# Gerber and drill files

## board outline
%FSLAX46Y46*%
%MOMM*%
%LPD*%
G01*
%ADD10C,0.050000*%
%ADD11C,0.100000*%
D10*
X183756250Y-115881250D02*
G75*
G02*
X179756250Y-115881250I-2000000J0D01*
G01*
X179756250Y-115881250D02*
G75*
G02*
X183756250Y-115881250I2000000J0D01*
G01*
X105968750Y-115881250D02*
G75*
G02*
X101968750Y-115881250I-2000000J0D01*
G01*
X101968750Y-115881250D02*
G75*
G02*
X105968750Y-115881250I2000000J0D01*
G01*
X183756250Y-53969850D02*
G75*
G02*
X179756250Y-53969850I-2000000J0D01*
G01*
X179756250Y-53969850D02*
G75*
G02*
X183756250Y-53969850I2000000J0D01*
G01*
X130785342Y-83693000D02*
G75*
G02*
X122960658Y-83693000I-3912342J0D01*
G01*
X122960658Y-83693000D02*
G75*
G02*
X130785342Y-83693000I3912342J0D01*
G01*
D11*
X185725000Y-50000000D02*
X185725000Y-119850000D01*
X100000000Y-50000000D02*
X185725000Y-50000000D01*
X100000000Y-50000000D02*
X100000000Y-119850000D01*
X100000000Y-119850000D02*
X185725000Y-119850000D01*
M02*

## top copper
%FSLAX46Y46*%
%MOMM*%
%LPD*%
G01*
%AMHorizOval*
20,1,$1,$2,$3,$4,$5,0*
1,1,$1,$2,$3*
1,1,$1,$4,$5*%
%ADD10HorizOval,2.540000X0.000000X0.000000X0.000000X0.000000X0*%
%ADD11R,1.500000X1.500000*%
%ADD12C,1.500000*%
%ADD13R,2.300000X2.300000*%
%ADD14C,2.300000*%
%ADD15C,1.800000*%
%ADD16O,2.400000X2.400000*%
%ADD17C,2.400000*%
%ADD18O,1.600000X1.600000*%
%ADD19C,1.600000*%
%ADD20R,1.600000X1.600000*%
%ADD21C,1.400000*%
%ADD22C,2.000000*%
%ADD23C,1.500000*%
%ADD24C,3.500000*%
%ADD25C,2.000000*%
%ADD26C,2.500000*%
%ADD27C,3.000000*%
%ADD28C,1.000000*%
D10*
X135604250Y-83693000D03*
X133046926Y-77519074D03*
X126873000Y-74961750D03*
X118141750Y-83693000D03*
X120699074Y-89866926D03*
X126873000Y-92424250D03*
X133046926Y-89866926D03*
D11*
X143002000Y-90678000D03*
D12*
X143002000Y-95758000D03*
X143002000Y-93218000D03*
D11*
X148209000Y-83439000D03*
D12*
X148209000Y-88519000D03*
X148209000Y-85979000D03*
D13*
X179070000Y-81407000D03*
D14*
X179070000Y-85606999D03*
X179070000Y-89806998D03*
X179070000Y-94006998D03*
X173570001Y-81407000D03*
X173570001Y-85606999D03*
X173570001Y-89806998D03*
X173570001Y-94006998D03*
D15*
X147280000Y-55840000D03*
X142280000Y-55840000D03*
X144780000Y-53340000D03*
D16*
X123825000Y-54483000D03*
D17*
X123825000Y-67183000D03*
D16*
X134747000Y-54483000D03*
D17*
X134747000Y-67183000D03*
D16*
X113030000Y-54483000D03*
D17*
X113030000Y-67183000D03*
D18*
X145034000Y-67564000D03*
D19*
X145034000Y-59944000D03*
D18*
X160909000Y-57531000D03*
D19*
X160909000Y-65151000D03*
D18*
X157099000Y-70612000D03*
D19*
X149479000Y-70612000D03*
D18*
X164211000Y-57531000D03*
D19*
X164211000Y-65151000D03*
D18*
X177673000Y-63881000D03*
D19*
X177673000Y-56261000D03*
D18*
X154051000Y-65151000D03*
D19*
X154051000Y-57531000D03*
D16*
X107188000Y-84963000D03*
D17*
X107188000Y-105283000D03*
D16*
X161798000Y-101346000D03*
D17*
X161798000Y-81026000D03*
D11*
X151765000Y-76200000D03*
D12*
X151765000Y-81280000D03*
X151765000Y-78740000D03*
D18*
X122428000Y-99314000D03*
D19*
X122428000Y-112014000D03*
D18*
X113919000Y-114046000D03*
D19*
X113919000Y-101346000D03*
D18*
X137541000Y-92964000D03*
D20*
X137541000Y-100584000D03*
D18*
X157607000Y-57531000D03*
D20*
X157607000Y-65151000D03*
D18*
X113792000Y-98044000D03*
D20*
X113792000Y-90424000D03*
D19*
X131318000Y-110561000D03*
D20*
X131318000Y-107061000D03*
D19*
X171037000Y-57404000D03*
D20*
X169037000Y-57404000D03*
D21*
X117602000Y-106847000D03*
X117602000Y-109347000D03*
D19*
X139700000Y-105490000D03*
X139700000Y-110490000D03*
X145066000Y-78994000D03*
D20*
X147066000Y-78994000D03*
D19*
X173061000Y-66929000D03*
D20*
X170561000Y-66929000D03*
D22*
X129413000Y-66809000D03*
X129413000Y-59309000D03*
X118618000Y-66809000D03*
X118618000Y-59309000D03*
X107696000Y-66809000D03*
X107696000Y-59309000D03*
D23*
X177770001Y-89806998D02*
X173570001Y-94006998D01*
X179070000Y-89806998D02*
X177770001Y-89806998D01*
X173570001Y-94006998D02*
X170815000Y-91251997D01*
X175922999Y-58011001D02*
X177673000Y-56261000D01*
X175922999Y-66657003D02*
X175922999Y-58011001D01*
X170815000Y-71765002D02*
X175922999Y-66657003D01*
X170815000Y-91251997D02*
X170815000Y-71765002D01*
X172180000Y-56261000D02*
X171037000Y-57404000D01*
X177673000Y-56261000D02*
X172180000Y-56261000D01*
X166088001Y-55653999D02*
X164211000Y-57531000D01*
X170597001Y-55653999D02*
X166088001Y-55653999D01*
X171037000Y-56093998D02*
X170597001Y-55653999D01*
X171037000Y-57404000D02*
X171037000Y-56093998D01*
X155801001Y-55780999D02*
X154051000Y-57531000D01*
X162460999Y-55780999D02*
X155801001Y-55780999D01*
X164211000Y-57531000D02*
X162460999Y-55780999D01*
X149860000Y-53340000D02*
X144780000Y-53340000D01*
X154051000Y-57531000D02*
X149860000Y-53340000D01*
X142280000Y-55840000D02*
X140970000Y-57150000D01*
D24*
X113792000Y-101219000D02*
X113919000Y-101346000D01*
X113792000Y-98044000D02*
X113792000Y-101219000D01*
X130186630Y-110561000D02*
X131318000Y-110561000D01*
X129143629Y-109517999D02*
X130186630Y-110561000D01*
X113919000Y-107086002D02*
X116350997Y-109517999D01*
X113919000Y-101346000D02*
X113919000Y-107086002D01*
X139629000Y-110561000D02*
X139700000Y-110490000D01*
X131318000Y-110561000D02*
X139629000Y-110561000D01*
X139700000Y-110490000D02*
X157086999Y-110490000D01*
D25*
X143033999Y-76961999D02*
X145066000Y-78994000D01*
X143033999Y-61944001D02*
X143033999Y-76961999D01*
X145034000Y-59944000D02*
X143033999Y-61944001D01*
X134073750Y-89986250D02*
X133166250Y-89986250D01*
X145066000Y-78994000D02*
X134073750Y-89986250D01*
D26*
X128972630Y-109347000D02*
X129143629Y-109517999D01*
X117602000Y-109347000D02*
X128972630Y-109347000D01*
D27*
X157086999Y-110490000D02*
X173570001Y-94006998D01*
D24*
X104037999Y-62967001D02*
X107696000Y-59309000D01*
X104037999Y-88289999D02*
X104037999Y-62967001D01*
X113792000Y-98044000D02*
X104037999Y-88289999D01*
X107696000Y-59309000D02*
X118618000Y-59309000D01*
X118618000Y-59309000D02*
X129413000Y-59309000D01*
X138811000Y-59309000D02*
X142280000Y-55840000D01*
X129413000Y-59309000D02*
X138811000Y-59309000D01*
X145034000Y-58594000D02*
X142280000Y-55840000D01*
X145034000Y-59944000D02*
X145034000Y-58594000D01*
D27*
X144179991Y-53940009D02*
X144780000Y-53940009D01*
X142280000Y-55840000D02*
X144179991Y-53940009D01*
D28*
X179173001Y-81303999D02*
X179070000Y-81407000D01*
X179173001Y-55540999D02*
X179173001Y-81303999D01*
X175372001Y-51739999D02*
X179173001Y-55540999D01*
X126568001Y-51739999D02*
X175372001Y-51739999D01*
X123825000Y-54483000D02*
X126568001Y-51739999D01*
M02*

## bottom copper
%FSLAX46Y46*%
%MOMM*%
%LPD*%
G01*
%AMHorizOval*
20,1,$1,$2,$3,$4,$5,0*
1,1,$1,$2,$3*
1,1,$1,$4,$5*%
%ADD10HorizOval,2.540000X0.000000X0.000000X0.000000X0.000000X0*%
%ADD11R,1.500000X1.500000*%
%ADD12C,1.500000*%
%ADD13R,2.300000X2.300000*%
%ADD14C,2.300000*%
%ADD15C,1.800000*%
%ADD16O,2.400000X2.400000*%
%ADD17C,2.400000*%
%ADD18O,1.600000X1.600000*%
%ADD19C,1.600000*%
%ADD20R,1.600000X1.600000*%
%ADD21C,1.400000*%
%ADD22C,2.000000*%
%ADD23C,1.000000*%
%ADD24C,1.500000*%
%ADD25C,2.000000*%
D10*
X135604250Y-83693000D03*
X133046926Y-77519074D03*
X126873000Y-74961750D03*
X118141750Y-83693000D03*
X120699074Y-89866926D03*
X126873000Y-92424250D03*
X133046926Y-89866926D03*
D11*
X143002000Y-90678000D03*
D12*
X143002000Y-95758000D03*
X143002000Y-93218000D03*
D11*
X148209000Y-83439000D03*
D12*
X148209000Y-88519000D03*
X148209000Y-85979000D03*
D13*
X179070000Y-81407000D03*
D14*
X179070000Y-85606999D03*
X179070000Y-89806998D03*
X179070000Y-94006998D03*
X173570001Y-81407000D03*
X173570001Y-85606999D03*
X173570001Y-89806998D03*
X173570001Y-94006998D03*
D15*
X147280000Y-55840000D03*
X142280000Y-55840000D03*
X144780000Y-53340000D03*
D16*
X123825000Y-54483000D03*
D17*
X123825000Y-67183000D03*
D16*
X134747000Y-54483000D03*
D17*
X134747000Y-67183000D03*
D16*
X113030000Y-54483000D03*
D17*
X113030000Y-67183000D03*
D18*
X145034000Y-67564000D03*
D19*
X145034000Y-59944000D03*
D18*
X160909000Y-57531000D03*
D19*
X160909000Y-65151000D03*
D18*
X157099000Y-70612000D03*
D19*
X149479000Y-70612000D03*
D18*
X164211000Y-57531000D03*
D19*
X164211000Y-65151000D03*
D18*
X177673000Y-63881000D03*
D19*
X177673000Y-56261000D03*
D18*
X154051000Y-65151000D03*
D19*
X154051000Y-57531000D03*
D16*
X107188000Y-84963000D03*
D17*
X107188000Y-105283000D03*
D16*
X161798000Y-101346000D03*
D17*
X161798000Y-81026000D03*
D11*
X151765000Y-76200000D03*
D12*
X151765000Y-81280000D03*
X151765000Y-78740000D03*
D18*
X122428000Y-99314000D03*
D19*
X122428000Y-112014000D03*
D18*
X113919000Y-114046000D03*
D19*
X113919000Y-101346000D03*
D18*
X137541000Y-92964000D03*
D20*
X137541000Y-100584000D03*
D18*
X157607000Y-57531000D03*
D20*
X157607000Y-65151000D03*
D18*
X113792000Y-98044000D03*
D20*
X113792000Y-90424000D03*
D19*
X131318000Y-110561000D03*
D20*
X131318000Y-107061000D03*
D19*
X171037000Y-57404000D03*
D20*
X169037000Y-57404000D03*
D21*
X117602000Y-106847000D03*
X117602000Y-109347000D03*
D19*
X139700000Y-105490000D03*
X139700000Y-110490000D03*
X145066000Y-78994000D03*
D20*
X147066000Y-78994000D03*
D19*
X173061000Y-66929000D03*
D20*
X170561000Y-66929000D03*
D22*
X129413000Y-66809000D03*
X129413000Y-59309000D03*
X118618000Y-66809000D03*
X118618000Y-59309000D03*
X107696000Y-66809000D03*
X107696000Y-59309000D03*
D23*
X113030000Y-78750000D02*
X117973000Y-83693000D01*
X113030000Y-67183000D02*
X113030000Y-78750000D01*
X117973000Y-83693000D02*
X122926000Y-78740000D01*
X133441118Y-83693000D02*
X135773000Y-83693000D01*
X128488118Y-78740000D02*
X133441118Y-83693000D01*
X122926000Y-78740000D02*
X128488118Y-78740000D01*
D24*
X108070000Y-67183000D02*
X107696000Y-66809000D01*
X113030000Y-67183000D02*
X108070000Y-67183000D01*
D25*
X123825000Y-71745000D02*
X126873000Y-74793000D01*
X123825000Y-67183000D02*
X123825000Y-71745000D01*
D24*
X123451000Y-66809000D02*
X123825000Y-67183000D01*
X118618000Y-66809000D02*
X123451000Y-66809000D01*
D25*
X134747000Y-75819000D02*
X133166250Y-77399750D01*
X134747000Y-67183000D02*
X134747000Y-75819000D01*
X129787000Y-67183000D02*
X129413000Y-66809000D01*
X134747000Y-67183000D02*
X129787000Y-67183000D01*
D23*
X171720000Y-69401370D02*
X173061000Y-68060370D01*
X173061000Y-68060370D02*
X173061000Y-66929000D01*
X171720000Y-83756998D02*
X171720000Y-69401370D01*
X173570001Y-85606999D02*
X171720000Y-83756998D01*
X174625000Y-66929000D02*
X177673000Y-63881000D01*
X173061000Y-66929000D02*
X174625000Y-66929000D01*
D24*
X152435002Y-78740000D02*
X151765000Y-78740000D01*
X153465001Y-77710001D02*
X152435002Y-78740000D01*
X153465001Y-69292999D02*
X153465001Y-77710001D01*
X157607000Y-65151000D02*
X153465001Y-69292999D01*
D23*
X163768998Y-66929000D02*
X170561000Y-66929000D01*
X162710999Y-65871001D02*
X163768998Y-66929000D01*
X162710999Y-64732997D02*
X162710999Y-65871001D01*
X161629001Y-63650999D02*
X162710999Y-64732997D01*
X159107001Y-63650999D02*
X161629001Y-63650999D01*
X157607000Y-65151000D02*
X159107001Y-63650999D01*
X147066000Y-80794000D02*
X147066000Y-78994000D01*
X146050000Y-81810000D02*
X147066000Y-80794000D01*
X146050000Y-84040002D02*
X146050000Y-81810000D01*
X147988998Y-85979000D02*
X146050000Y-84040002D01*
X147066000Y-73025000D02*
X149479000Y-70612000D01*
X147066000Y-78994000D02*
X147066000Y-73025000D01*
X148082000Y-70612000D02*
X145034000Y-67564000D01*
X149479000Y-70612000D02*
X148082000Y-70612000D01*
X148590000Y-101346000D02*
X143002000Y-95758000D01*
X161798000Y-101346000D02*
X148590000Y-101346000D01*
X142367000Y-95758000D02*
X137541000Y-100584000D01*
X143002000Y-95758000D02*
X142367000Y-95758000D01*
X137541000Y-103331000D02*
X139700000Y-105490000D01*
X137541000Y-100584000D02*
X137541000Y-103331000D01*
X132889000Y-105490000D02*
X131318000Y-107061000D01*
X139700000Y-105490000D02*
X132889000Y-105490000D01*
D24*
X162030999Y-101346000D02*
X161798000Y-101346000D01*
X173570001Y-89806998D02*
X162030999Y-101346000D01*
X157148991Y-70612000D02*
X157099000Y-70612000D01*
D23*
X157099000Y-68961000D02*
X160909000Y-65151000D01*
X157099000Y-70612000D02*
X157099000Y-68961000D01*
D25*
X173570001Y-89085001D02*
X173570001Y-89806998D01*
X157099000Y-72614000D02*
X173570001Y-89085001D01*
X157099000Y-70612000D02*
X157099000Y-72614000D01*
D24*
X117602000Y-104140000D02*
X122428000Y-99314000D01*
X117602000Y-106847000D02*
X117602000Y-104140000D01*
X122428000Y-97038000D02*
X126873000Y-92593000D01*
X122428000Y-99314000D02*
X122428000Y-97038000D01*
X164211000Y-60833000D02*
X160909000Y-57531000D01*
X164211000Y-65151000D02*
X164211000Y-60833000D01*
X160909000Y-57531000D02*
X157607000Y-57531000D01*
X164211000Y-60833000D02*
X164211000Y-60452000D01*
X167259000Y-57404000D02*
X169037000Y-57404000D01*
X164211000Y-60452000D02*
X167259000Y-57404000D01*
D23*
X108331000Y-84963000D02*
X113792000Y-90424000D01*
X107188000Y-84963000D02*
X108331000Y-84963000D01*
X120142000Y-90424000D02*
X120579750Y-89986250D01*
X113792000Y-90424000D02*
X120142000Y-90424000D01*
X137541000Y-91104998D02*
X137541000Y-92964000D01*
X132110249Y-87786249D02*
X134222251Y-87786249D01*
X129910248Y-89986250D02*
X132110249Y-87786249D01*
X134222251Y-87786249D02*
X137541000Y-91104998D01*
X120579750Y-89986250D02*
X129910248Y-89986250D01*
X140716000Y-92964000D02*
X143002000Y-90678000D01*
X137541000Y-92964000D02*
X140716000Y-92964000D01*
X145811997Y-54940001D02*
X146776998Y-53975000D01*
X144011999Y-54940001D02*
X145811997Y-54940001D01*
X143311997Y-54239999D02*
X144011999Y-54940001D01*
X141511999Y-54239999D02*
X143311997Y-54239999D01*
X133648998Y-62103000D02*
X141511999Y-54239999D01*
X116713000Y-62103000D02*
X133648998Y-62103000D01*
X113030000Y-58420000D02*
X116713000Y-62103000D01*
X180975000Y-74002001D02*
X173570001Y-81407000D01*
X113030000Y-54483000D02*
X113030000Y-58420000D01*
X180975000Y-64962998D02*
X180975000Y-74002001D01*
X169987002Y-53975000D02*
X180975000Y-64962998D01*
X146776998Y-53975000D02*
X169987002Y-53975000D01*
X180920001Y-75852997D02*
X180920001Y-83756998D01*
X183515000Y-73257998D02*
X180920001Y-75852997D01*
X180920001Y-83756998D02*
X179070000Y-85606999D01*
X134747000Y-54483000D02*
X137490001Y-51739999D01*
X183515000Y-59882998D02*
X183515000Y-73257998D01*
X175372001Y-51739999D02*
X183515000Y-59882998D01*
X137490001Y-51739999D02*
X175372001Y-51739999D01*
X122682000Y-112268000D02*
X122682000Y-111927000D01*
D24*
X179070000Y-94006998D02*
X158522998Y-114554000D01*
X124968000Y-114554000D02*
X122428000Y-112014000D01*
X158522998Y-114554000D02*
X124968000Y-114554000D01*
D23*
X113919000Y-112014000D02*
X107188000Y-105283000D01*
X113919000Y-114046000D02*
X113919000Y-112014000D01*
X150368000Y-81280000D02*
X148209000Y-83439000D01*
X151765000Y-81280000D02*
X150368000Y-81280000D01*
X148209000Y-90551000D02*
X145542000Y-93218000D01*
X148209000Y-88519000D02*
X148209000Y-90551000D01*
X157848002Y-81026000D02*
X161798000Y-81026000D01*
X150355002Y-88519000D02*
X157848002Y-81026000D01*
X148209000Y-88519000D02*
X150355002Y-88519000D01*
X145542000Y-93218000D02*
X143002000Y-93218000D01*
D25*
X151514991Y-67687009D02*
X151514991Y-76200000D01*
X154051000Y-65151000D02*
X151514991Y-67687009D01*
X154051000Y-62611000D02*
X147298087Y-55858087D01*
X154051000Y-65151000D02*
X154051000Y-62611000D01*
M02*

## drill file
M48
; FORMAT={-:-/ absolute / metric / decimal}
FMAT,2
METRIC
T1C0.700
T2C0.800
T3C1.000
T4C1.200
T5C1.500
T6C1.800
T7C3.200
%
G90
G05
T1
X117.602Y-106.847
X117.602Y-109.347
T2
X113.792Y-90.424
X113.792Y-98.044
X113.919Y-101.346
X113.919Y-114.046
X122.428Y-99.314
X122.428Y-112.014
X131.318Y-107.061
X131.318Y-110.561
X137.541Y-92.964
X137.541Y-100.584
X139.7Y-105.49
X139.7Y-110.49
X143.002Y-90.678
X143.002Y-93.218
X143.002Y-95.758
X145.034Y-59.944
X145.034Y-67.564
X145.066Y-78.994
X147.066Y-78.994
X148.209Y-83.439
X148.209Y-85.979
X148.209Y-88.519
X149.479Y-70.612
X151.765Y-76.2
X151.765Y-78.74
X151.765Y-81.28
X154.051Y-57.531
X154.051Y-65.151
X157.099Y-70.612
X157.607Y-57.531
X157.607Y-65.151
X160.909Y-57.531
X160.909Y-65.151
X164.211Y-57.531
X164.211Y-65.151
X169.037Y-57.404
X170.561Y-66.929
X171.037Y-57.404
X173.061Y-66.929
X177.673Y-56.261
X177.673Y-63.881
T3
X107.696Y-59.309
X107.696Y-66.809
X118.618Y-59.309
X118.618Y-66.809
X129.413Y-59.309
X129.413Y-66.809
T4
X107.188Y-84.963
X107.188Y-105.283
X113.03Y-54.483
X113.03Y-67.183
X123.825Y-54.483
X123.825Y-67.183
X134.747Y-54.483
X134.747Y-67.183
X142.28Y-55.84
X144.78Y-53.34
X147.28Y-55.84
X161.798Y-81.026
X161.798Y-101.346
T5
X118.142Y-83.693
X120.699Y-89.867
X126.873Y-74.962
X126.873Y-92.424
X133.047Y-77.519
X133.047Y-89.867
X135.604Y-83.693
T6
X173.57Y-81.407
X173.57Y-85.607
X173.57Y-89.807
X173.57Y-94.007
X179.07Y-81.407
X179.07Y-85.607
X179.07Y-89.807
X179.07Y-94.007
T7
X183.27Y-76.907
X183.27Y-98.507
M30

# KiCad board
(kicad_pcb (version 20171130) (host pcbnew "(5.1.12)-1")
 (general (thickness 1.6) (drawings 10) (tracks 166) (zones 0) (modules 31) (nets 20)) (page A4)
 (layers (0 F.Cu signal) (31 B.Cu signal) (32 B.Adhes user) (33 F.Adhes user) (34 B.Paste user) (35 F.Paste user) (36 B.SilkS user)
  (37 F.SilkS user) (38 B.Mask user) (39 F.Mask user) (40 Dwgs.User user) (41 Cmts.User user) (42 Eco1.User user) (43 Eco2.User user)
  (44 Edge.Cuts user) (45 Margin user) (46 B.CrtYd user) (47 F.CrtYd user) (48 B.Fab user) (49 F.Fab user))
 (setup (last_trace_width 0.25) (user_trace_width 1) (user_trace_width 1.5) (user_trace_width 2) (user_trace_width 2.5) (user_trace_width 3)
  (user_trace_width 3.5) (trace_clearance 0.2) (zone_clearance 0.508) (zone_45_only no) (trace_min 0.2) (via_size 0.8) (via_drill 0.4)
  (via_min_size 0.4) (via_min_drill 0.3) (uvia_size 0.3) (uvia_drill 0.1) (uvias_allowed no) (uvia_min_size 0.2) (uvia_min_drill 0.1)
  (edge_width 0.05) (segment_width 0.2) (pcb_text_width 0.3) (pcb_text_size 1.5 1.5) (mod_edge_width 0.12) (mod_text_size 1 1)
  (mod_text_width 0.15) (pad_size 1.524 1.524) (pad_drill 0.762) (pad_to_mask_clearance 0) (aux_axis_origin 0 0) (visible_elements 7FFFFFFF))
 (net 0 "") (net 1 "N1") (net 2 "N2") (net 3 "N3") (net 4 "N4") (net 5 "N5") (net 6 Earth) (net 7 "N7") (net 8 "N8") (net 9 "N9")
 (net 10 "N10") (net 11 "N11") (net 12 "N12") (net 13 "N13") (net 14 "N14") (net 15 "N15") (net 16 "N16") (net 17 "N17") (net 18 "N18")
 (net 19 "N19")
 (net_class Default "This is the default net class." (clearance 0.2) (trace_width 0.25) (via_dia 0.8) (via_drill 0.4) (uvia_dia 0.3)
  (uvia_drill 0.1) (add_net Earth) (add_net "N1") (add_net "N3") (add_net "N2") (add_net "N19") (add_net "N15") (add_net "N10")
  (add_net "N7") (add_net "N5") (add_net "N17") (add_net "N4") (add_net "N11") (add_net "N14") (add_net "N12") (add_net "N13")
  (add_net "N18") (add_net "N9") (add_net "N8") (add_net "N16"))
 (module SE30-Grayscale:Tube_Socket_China (layer F.Cu) (at 126.873 83.693 225)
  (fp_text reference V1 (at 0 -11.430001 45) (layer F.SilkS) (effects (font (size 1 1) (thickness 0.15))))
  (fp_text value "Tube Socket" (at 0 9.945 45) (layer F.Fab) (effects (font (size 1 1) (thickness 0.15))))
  (pad 5 thru_hole oval (at -6.173926 -6.173926 225) (size 2.54 2.54) (drill 1.5) (layers *.Cu *.Mask) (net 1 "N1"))
  (pad 6 thru_hole oval (at -8.73125 0 225) (size 2.54 2.54) (drill 1.5) (layers *.Cu *.Mask) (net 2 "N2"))
  (pad 7 thru_hole oval (at -6.173926 6.173926 225) (size 2.54 2.54) (drill 1.5) (layers *.Cu *.Mask) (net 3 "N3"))
  (pad 1 thru_hole oval (at 6.173926 6.173926 225) (size 2.54 2.54) (drill 1.5) (layers *.Cu *.Mask) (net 1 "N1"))
  (pad 2 thru_hole oval (at 8.73125 0 225) (size 2.54 2.54) (drill 1.5) (layers *.Cu *.Mask) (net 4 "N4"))
  (pad 3 thru_hole oval (at 6.173926 -6.173926 225) (size 2.54 2.54) (drill 1.5) (layers *.Cu *.Mask) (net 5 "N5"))
  (pad 4 thru_hole oval (at 0 -8.73125 225) (size 2.54 2.54) (drill 1.5) (layers *.Cu *.Mask) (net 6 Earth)))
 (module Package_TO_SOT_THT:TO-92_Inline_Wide (layer F.Cu) (at 143.002 90.678 270)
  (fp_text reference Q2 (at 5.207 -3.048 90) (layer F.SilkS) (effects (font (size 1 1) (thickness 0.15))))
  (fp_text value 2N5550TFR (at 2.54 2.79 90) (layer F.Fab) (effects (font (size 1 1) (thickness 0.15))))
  (pad 1 thru_hole rect (at 0 0 270) (size 1.5 1.5) (drill 0.8) (layers *.Cu *.Mask) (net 4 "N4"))
  (pad 3 thru_hole circle (at 5.08 0 270) (size 1.5 1.5) (drill 0.8) (layers *.Cu *.Mask) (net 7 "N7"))
  (pad 2 thru_hole circle (at 2.54 0 270) (size 1.5 1.5) (drill 0.8) (layers *.Cu *.Mask) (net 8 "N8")))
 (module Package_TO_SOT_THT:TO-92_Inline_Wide (layer F.Cu) (at 148.209 83.439 270)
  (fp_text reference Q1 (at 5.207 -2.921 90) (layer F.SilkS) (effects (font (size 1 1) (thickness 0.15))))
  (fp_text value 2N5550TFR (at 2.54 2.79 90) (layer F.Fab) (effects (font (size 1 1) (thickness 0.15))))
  (pad 1 thru_hole rect (at 0 0 270) (size 1.5 1.5) (drill 0.8) (layers *.Cu *.Mask) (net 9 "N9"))
  (pad 3 thru_hole circle (at 5.08 0 270) (size 1.5 1.5) (drill 0.8) (layers *.Cu *.Mask) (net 8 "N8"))
  (pad 2 thru_hole circle (at 2.54 0 270) (size 1.5 1.5) (drill 0.8) (layers *.Cu *.Mask) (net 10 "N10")))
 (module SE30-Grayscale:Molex (layer F.Cu) (at 179.07 81.407 90)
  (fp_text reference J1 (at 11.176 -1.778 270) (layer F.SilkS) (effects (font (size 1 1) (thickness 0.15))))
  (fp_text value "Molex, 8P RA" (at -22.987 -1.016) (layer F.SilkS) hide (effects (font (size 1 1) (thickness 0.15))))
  (pad 1 thru_hole rect (at 0 0 90) (size 2.3 2.3) (drill 1.8) (layers *.Cu *.Mask) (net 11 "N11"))
  (pad 3 thru_hole circle (at -4.199999 0 90) (size 2.3 2.3) (drill 1.8) (layers *.Cu *.Mask) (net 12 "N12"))
  (pad 5 thru_hole circle (at -8.399998 0 90) (size 2.3 2.3) (drill 1.8) (layers *.Cu *.Mask) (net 6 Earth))
  (pad 7 thru_hole circle (at -12.599998 0 90) (size 2.3 2.3) (drill 1.8) (layers *.Cu *.Mask) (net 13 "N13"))
  (pad 2 thru_hole circle (at 0 -5.499999 90) (size 2.3 2.3) (drill 1.8) (layers *.Cu *.Mask) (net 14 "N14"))
  (pad 4 thru_hole circle (at -4.199999 -5.499999 90) (size 2.3 2.3) (drill 1.8) (layers *.Cu *.Mask) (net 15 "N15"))
  (pad 6 thru_hole circle (at -8.399998 -5.499999 90) (size 2.3 2.3) (drill 1.8) (layers *.Cu *.Mask) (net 7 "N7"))
  (pad 8 thru_hole circle (at -12.599998 -5.499999 90) (size 2.3 2.3) (drill 1.8) (layers *.Cu *.Mask) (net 6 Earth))
  (pad M1 np_thru_hole circle (at 4.499999 4.199999 90) (size 3.200001 3.200001) (drill 3.200001) (layers *.Cu *.Mask))
  (pad M2 np_thru_hole circle (at -17.099958 4.199999 90) (size 3.200001 3.200001) (drill 3.200001) (layers *.Cu *.Mask)))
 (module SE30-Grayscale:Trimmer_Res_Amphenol (layer F.Cu) (at 144.78 53.34)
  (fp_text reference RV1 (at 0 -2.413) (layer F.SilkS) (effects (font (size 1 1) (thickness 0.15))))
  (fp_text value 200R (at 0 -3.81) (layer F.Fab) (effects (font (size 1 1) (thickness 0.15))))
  (pad 3 thru_hole circle (at 2.5 2.5) (size 1.8 1.8) (drill 1.2) (layers *.Cu *.Mask) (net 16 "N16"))
  (pad 1 thru_hole circle (at -2.5 2.5) (size 1.8 1.8) (drill 1.2) (layers *.Cu *.Mask) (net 6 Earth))
  (pad 2 thru_hole circle (at 0 0) (size 1.8 1.8) (drill 1.2) (layers *.Cu *.Mask) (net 6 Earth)))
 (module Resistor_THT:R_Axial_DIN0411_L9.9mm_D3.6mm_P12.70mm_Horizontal (layer F.Cu) (at 123.825 67.183 90)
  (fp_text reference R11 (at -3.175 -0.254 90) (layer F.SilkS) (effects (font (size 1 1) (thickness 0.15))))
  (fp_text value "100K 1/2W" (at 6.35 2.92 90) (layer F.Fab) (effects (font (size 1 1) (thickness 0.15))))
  (pad 2 thru_hole oval (at 12.7 0 90) (size 2.4 2.4) (drill 1.2) (layers *.Cu *.Mask) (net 11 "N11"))
  (pad 1 thru_hole circle (at 0 0 90) (size 2.4 2.4) (drill 1.2) (layers *.Cu *.Mask) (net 3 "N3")))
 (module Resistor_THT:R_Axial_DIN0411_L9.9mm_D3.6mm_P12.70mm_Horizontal (layer F.Cu) (at 134.747 67.183 90)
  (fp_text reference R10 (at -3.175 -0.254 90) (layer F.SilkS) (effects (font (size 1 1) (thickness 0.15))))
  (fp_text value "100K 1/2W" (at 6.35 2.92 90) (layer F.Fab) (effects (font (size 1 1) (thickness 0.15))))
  (pad 2 thru_hole oval (at 12.7 0 90) (size 2.4 2.4) (drill 1.2) (layers *.Cu *.Mask) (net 12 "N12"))
  (pad 1 thru_hole circle (at 0 0 90) (size 2.4 2.4) (drill 1.2) (layers *.Cu *.Mask) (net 2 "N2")))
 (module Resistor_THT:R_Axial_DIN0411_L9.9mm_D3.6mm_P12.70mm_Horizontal (layer F.Cu) (at 113.03 67.183 90)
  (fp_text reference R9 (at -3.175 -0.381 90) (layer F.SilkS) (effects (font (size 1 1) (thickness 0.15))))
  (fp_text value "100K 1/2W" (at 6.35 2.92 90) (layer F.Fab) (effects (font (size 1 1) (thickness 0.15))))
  (pad 2 thru_hole oval (at 12.7 0 90) (size 2.4 2.4) (drill 1.2) (layers *.Cu *.Mask) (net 14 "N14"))
  (pad 1 thru_hole circle (at 0 0 90) (size 2.4 2.4) (drill 1.2) (layers *.Cu *.Mask) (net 1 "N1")))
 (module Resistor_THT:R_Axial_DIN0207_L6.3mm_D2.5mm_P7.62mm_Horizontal (layer F.Cu) (at 145.034 59.944 270)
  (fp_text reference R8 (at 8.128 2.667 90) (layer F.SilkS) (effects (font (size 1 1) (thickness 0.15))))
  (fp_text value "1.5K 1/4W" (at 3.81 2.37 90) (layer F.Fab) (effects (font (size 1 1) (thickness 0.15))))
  (pad 2 thru_hole oval (at 7.62 0 270) (size 1.6 1.6) (drill 0.8) (layers *.Cu *.Mask) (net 10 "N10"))
  (pad 1 thru_hole circle (at 0 0 270) (size 1.6 1.6) (drill 0.8) (layers *.Cu *.Mask) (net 6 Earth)))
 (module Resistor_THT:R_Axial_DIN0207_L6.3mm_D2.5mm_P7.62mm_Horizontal (layer F.Cu) (at 160.909 65.151 90)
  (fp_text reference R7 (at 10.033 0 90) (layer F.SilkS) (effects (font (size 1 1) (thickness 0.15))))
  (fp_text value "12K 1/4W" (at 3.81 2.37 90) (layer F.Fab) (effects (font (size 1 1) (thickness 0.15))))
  (pad 2 thru_hole oval (at 7.62 0 90) (size 1.6 1.6) (drill 0.8) (layers *.Cu *.Mask) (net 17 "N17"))
  (pad 1 thru_hole circle (at 0 0 90) (size 1.6 1.6) (drill 0.8) (layers *.Cu *.Mask) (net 7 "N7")))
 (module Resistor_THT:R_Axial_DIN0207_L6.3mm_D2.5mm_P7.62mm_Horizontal (layer F.Cu) (at 149.479 70.612)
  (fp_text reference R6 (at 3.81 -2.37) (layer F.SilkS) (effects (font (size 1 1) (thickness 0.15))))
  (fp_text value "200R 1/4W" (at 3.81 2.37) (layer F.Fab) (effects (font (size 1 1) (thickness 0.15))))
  (pad 2 thru_hole oval (at 7.62 0) (size 1.6 1.6) (drill 0.8) (layers *.Cu *.Mask) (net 7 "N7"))
  (pad 1 thru_hole circle (at 0 0) (size 1.6 1.6) (drill 0.8) (layers *.Cu *.Mask) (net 10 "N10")))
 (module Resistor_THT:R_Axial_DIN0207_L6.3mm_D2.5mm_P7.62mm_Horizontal (layer F.Cu) (at 164.211 65.151 90)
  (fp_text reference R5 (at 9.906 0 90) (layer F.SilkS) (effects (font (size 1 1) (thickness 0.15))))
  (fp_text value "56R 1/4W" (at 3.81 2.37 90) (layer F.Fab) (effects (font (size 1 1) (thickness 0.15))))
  (pad 2 thru_hole oval (at 7.62 0 90) (size 1.6 1.6) (drill 0.8) (layers *.Cu *.Mask) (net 6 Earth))
  (pad 1 thru_hole circle (at 0 0 90) (size 1.6 1.6) (drill 0.8) (layers *.Cu *.Mask) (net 17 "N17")))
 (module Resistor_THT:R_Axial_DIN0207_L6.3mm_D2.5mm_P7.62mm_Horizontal (layer F.Cu) (at 177.673 56.261 270)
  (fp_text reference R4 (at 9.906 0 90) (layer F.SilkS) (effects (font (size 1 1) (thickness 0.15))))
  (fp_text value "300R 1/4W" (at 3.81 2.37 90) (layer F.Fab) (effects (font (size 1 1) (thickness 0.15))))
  (pad 2 thru_hole oval (at 7.62 0 270) (size 1.6 1.6) (drill 0.8) (layers *.Cu *.Mask) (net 15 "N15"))
  (pad 1 thru_hole circle (at 0 0 270) (size 1.6 1.6) (drill 0.8) (layers *.Cu *.Mask) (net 6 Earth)))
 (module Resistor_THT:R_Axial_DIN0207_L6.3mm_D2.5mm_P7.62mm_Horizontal (layer F.Cu) (at 154.051 57.531 270)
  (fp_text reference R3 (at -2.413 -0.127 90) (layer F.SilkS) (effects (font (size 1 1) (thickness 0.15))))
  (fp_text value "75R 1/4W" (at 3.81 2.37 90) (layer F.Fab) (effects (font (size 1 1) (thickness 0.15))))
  (pad 2 thru_hole oval (at 7.62 0 270) (size 1.6 1.6) (drill 0.8) (layers *.Cu *.Mask) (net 16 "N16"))
  (pad 1 thru_hole circle (at 0 0 270) (size 1.6 1.6) (drill 0.8) (layers *.Cu *.Mask) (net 6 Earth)))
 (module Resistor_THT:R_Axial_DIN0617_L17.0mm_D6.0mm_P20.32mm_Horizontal (layer F.Cu) (at 107.188 105.283 90)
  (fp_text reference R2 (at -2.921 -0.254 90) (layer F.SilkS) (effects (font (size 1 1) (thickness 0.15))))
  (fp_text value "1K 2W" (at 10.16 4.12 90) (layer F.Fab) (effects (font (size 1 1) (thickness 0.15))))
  (pad 2 thru_hole oval (at 20.32 0 90) (size 2.4 2.4) (drill 1.2) (layers *.Cu *.Mask) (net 4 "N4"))
  (pad 1 thru_hole circle (at 0 0 90) (size 2.4 2.4) (drill 1.2) (layers *.Cu *.Mask) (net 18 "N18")))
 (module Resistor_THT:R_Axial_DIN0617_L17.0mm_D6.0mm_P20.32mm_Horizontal (layer F.Cu) (at 161.798 81.026 270)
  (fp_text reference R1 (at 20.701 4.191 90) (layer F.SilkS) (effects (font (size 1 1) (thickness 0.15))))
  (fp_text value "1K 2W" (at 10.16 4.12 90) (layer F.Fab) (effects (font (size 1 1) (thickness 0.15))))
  (pad 2 thru_hole oval (at 20.32 0 270) (size 2.4 2.4) (drill 1.2) (layers *.Cu *.Mask) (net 7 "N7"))
  (pad 1 thru_hole circle (at 0 0 270) (size 2.4 2.4) (drill 1.2) (layers *.Cu *.Mask) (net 8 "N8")))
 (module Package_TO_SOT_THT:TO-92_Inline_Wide (layer F.Cu) (at 151.765 76.2 270)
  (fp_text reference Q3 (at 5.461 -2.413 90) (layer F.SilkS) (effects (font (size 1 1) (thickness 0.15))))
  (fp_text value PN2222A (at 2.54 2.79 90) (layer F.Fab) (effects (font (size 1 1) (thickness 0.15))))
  (pad 1 thru_hole rect (at 0 0 270) (size 1.5 1.5) (drill 0.8) (layers *.Cu *.Mask) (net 16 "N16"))
  (pad 3 thru_hole circle (at 5.08 0 270) (size 1.5 1.5) (drill 0.8) (layers *.Cu *.Mask) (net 9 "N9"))
  (pad 2 thru_hole circle (at 2.54 0 270) (size 1.5 1.5) (drill 0.8) (layers *.Cu *.Mask) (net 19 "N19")))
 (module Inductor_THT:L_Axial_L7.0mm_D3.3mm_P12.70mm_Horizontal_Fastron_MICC (layer F.Cu) (at 122.428 112.014 90)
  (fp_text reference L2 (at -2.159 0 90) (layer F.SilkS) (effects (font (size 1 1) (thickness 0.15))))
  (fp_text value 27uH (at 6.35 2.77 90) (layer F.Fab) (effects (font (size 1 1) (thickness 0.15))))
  (pad 2 thru_hole oval (at 12.7 0 90) (size 1.6 1.6) (drill 0.8) (layers *.Cu *.Mask) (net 5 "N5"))
  (pad 1 thru_hole circle (at 0 0 90) (size 1.6 1.6) (drill 0.8) (layers *.Cu *.Mask) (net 13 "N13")))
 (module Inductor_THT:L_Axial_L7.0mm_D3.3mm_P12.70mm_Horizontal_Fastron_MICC (layer F.Cu) (at 113.919 101.346 270)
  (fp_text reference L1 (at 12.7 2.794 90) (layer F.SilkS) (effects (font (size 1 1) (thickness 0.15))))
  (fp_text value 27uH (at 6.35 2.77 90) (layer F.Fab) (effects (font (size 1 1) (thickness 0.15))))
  (pad 2 thru_hole oval (at 12.7 0 270) (size 1.6 1.6) (drill 0.8) (layers *.Cu *.Mask) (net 18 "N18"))
  (pad 1 thru_hole circle (at 0 0 270) (size 1.6 1.6) (drill 0.8) (layers *.Cu *.Mask) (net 6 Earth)))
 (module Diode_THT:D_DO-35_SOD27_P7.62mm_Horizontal (layer F.Cu) (at 137.541 100.584 90)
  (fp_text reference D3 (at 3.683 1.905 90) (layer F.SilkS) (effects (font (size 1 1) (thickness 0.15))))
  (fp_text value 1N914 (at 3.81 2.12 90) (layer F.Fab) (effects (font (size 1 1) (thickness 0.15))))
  (pad 2 thru_hole oval (at 7.62 0 90) (size 1.6 1.6) (drill 0.8) (layers *.Cu *.Mask) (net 4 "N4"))
  (pad 1 thru_hole rect (at 0 0 90) (size 1.6 1.6) (drill 0.8) (layers *.Cu *.Mask) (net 7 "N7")))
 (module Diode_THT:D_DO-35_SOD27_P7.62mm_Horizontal (layer F.Cu) (at 157.607 65.151 90)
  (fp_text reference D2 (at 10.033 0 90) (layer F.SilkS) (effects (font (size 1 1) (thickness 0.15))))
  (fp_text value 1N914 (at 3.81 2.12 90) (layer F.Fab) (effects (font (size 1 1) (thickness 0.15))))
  (pad 2 thru_hole oval (at 7.62 0 90) (size 1.6 1.6) (drill 0.8) (layers *.Cu *.Mask) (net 17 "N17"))
  (pad 1 thru_hole rect (at 0 0 90) (size 1.6 1.6) (drill 0.8) (layers *.Cu *.Mask) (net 19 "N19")))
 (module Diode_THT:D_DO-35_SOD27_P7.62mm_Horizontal (layer F.Cu) (at 113.792 90.424 270)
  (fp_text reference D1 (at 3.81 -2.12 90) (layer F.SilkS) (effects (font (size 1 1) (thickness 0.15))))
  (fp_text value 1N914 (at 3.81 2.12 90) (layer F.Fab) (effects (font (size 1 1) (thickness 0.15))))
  (pad 2 thru_hole oval (at 7.62 0 270) (size 1.6 1.6) (drill 0.8) (layers *.Cu *.Mask) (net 6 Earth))
  (pad 1 thru_hole rect (at 0 0 270) (size 1.6 1.6) (drill 0.8) (layers *.Cu *.Mask) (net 4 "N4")))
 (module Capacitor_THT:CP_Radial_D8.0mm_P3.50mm (layer F.Cu) (at 131.318 107.061 270)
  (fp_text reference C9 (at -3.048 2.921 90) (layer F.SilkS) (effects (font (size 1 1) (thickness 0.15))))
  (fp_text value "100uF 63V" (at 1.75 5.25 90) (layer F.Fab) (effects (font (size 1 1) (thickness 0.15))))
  (pad 2 thru_hole circle (at 3.5 0 270) (size 1.6 1.6) (drill 0.8) (layers *.Cu *.Mask) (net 6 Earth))
  (pad 1 thru_hole rect (at 0 0 270) (size 1.6 1.6) (drill 0.8) (layers *.Cu *.Mask) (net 7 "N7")))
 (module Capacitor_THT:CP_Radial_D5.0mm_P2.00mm (layer F.Cu) (at 169.037 57.404)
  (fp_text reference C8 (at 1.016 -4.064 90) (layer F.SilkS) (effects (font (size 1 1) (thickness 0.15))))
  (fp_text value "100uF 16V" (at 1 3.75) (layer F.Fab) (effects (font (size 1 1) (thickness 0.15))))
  (pad 2 thru_hole circle (at 2 0) (size 1.6 1.6) (drill 0.8) (layers *.Cu *.Mask) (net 6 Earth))
  (pad 1 thru_hole rect (at 0 0) (size 1.6 1.6) (drill 0.8) (layers *.Cu *.Mask) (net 17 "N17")))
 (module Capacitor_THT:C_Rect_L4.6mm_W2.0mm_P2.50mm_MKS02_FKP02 (layer F.Cu) (at 117.602 109.347 90)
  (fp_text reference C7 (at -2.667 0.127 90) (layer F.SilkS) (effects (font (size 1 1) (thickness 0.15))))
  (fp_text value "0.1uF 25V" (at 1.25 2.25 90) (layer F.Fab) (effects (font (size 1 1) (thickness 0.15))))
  (pad 2 thru_hole circle (at 2.5 0 90) (size 1.4 1.4) (drill 0.7) (layers *.Cu *.Mask) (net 5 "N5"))
  (pad 1 thru_hole circle (at 0 0 90) (size 1.4 1.4) (drill 0.7) (layers *.Cu *.Mask) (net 6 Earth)))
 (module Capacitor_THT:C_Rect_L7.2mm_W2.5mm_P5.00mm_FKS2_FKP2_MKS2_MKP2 (layer F.Cu) (at 139.7 110.49 90)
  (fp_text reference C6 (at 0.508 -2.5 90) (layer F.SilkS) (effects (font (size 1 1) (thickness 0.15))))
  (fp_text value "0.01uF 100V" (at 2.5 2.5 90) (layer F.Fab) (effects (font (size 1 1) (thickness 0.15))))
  (pad 2 thru_hole circle (at 5 0 90) (size 1.6 1.6) (drill 0.8) (layers *.Cu *.Mask) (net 7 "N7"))
  (pad 1 thru_hole circle (at 0 0 90) (size 1.6 1.6) (drill 0.8) (layers *.Cu *.Mask) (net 6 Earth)))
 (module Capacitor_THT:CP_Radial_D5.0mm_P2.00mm (layer F.Cu) (at 147.066 78.994 180)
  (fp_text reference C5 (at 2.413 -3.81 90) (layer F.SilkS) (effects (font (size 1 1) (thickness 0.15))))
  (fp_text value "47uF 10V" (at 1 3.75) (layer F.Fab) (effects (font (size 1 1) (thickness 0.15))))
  (pad 2 thru_hole circle (at 2 0 180) (size 1.6 1.6) (drill 0.8) (layers *.Cu *.Mask) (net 6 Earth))
  (pad 1 thru_hole rect (at 0 0 180) (size 1.6 1.6) (drill 0.8) (layers *.Cu *.Mask) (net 10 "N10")))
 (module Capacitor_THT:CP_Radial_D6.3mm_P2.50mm (layer F.Cu) (at 170.561 66.929)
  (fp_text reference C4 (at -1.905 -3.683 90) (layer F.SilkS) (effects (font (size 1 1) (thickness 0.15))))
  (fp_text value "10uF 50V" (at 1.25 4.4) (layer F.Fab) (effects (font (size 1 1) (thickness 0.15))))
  (pad 2 thru_hole circle (at 2.5 0) (size 1.6 1.6) (drill 0.8) (layers *.Cu *.Mask) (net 15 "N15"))
  (pad 1 thru_hole rect (at 0 0) (size 1.6 1.6) (drill 0.8) (layers *.Cu *.Mask) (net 19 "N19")))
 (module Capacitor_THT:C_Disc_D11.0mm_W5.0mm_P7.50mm (layer F.Cu) (at 129.413 59.309 270)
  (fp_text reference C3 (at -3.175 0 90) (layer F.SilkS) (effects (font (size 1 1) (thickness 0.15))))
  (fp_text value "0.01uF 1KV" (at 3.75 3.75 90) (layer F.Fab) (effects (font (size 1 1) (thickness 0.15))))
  (pad 2 thru_hole circle (at 7.5 0 270) (size 2 2) (drill 1) (layers *.Cu *.Mask) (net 2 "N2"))
  (pad 1 thru_hole circle (at 0 0 270) (size 2 2) (drill 1) (layers *.Cu *.Mask) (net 6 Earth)))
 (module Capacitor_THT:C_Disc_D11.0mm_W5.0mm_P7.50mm (layer F.Cu) (at 118.618 59.309 270)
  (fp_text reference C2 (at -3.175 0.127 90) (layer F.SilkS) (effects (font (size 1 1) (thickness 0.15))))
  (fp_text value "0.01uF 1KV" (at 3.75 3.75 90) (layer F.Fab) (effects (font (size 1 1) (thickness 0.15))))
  (pad 2 thru_hole circle (at 7.5 0 270) (size 2 2) (drill 1) (layers *.Cu *.Mask) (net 3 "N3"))
  (pad 1 thru_hole circle (at 0 0 270) (size 2 2) (drill 1) (layers *.Cu *.Mask) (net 6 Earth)))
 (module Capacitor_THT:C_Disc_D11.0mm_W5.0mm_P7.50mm (layer F.Cu) (at 107.696 59.309 270)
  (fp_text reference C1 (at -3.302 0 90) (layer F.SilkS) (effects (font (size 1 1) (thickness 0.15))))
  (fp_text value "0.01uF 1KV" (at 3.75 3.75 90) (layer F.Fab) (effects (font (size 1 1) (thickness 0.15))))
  (pad 2 thru_hole circle (at 7.5 0 270) (size 2 2) (drill 1) (layers *.Cu *.Mask) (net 1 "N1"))
  (pad 1 thru_hole circle (at 0 0 270) (size 2 2) (drill 1) (layers *.Cu *.Mask) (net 6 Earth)))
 (gr_circle (center 181.75625 115.88125) (end 183.75625 115.88125) (layer Edge.Cuts) (width 0.05))
 (gr_circle (center 103.96875 115.88125) (end 105.96875 115.88125) (layer Edge.Cuts) (width 0.05))
 (gr_circle (center 181.75625 53.96985) (end 183.75625 53.96985) (layer Edge.Cuts) (width 0.05))
 (gr_circle (center 126.873 83.693) (end 130.785342 83.693) (layer Edge.Cuts) (width 0.05))
 (gr_line (start 185.725 50) (end 185.725 119.85) (layer Edge.Cuts) (width 0.1))
 (gr_line (start 100 50) (end 185.725 50) (layer Edge.Cuts) (width 0.1))
 (gr_line (start 100 50) (end 100 119.85) (layer Edge.Cuts) (width 0.1))
 (gr_line (start 100 119.85) (end 185.725 119.85) (layer Edge.Cuts) (width 0.1))
 (segment (start 113.03 78.75) (end 117.973 83.693) (width 1) (layer B.Cu) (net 1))
 (segment (start 113.03 67.183) (end 113.03 78.75) (width 1) (layer B.Cu) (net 1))
 (segment (start 117.973 83.693) (end 122.926 78.74) (width 1) (layer B.Cu) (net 1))
 (segment (start 133.441118 83.693) (end 135.773 83.693) (width 1) (layer B.Cu) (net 1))
 (segment (start 128.488118 78.74) (end 133.441118 83.693) (width 1) (layer B.Cu) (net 1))
 (segment (start 122.926 78.74) (end 128.488118 78.74) (width 1) (layer B.Cu) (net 1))
 (segment (start 108.07 67.183) (end 107.696 66.809) (width 1.5) (layer B.Cu) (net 1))
 (segment (start 113.03 67.183) (end 108.07 67.183) (width 1.5) (layer B.Cu) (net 1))
 (segment (start 177.770001 89.806998) (end 173.570001 94.006998) (width 1.5) (layer F.Cu) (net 6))
 (segment (start 179.07 89.806998) (end 177.770001 89.806998) (width 1.5) (layer F.Cu) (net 6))
 (segment (start 173.570001 94.006998) (end 170.815 91.251997) (width 1.5) (layer F.Cu) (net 6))
 (segment (start 175.922999 58.011001) (end 177.673 56.261) (width 1.5) (layer F.Cu) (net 6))
 (segment (start 175.922999 66.657003) (end 175.922999 58.011001) (width 1.5) (layer F.Cu) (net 6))
 (segment (start 170.815 71.765002) (end 175.922999 66.657003) (width 1.5) (layer F.Cu) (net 6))
 (segment (start 170.815 91.251997) (end 170.815 71.765002) (width 1.5) (layer F.Cu) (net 6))
 (segment (start 172.18 56.261) (end 171.037 57.404) (width 1.5) (layer F.Cu) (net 6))
 (segment (start 177.673 56.261) (end 172.18 56.261) (width 1.5) (layer F.Cu) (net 6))
 (segment (start 166.088001 55.653999) (end 164.211 57.531) (width 1.5) (layer F.Cu) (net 6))
 (segment (start 170.597001 55.653999) (end 166.088001 55.653999) (width 1.5) (layer F.Cu) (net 6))
 (segment (start 171.037 56.093998) (end 170.597001 55.653999) (width 1.5) (layer F.Cu) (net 6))
 (segment (start 171.037 57.404) (end 171.037 56.093998) (width 1.5) (layer F.Cu) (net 6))
 (segment (start 155.801001 55.780999) (end 154.051 57.531) (width 1.5) (layer F.Cu) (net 6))
 (segment (start 162.460999 55.780999) (end 155.801001 55.780999) (width 1.5) (layer F.Cu) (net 6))
 (segment (start 164.211 57.531) (end 162.460999 55.780999) (width 1.5) (layer F.Cu) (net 6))
 (segment (start 149.86 53.34) (end 144.78 53.34) (width 1.5) (layer F.Cu) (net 6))
 (segment (start 154.051 57.531) (end 149.86 53.34) (width 1.5) (layer F.Cu) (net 6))
 (segment (start 142.28 55.84) (end 140.97 57.15) (width 1.5) (layer F.Cu) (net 6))
 (segment (start 113.792 101.219) (end 113.919 101.346) (width 3.5) (layer F.Cu) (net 6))
 (segment (start 113.792 98.044) (end 113.792 101.219) (width 3.5) (layer F.Cu) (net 6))
 (segment (start 130.18663 110.561) (end 131.318 110.561) (width 3.5) (layer F.Cu) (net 6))
 (segment (start 129.143629 109.517999) (end 130.18663 110.561) (width 3.5) (layer F.Cu) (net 6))
 (segment (start 113.919 107.086002) (end 116.350997 109.517999) (width 3.5) (layer F.Cu) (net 6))
 (segment (start 113.919 101.346) (end 113.919 107.086002) (width 3.5) (layer F.Cu) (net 6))
 (segment (start 139.629 110.561) (end 139.7 110.49) (width 3.5) (layer F.Cu) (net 6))
 (segment (start 131.318 110.561) (end 139.629 110.561) (width 3.5) (layer F.Cu) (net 6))
 (segment (start 139.7 110.49) (end 157.086999 110.49) (width 3.5) (layer F.Cu) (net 6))
 (segment (start 143.033999 76.961999) (end 145.066 78.994) (width 2) (layer F.Cu) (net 6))
 (segment (start 143.033999 61.944001) (end 143.033999 76.961999) (width 2) (layer F.Cu) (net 6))
 (segment (start 145.034 59.944) (end 143.033999 61.944001) (width 2) (layer F.Cu) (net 6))
 (segment (start 134.07375 89.98625) (end 133.16625 89.98625) (width 2) (layer F.Cu) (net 6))
 (segment (start 145.066 78.994) (end 134.07375 89.98625) (width 2) (layer F.Cu) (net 6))
 (segment (start 128.97263 109.347) (end 129.143629 109.517999) (width 2.5) (layer F.Cu) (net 6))
 (segment (start 117.602 109.347) (end 128.97263 109.347) (width 2.5) (layer F.Cu) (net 6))
 (segment (start 157.086999 110.49) (end 173.570001 94.006998) (width 3) (layer F.Cu) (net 6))
 (segment (start 104.037999 62.967001) (end 107.696 59.309) (width 3.5) (layer F.Cu) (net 6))
 (segment (start 104.037999 88.289999) (end 104.037999 62.967001) (width 3.5) (layer F.Cu) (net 6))
 (segment (start 113.792 98.044) (end 104.037999 88.289999) (width 3.5) (layer F.Cu) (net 6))
 (segment (start 107.696 59.309) (end 118.618 59.309) (width 3.5) (layer F.Cu) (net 6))
 (segment (start 118.618 59.309) (end 129.413 59.309) (width 3.5) (layer F.Cu) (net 6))
 (segment (start 138.811 59.309) (end 142.28 55.84) (width 3.5) (layer F.Cu) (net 6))
 (segment (start 129.413 59.309) (end 138.811 59.309) (width 3.5) (layer F.Cu) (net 6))
 (segment (start 145.034 58.594) (end 142.28 55.84) (width 3.5) (layer F.Cu) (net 6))
 (segment (start 145.034 59.944) (end 145.034 58.594) (width 3.5) (layer F.Cu) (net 6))
 (segment (start 144.179991 53.940009) (end 144.78 53.940009) (width 3) (layer F.Cu) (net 6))
 (segment (start 142.28 55.84) (end 144.179991 53.940009) (width 3) (layer F.Cu) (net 6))
 (segment (start 123.825 71.745) (end 126.873 74.793) (width 2) (layer B.Cu) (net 3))
 (segment (start 123.825 67.183) (end 123.825 71.745) (width 2) (layer B.Cu) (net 3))
 (segment (start 123.451 66.809) (end 123.825 67.183) (width 1.5) (layer B.Cu) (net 3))
 (segment (start 118.618 66.809) (end 123.451 66.809) (width 1.5) (layer B.Cu) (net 3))
 (segment (start 134.747 75.819) (end 133.16625 77.39975) (width 2) (layer B.Cu) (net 2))
 (segment (start 134.747 67.183) (end 134.747 75.819) (width 2) (layer B.Cu) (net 2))
 (segment (start 129.787 67.183) (end 129.413 66.809) (width 2) (layer B.Cu) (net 2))
 (segment (start 134.747 67.183) (end 129.787 67.183) (width 2) (layer B.Cu) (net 2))
 (segment (start 171.72 69.40137) (end 173.061 68.06037) (width 1) (layer B.Cu) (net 15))
 (segment (start 173.061 68.06037) (end 173.061 66.929) (width 1) (layer B.Cu) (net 15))
 (segment (start 171.72 83.756998) (end 171.72 69.40137) (width 1) (layer B.Cu) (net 15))
 (segment (start 173.570001 85.606999) (end 171.72 83.756998) (width 1) (layer B.Cu) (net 15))
 (segment (start 174.625 66.929) (end 177.673 63.881) (width 1) (layer B.Cu) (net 15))
 (segment (start 173.061 66.929) (end 174.625 66.929) (width 1) (layer B.Cu) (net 15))
 (segment (start 152.435002 78.74) (end 151.765 78.74) (width 1.5) (layer B.Cu) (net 19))
 (segment (start 153.465001 77.710001) (end 152.435002 78.74) (width 1.5) (layer B.Cu) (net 19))
 (segment (start 153.465001 69.292999) (end 153.465001 77.710001) (width 1.5) (layer B.Cu) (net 19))
 (segment (start 157.607 65.151) (end 153.465001 69.292999) (width 1.5) (layer B.Cu) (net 19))
 (segment (start 163.768998 66.929) (end 170.561 66.929) (width 1) (layer B.Cu) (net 19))
 (segment (start 162.710999 65.871001) (end 163.768998 66.929) (width 1) (layer B.Cu) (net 19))
 (segment (start 162.710999 64.732997) (end 162.710999 65.871001) (width 1) (layer B.Cu) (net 19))
 (segment (start 161.629001 63.650999) (end 162.710999 64.732997) (width 1) (layer B.Cu) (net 19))
 (segment (start 159.107001 63.650999) (end 161.629001 63.650999) (width 1) (layer B.Cu) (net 19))
 (segment (start 157.607 65.151) (end 159.107001 63.650999) (width 1) (layer B.Cu) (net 19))
 (segment (start 147.066 80.794) (end 147.066 78.994) (width 1) (layer B.Cu) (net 10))
 (segment (start 146.05 81.81) (end 147.066 80.794) (width 1) (layer B.Cu) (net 10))
 (segment (start 146.05 84.040002) (end 146.05 81.81) (width 1) (layer B.Cu) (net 10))
 (segment (start 147.988998 85.979) (end 146.05 84.040002) (width 1) (layer B.Cu) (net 10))
 (segment (start 147.066 73.025) (end 149.479 70.612) (width 1) (layer B.Cu) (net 10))
 (segment (start 147.066 78.994) (end 147.066 73.025) (width 1) (layer B.Cu) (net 10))
 (segment (start 148.082 70.612) (end 145.034 67.564) (width 1) (layer B.Cu) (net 10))
 (segment (start 149.479 70.612) (end 148.082 70.612) (width 1) (layer B.Cu) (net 10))
 (segment (start 148.59 101.346) (end 143.002 95.758) (width 1) (layer B.Cu) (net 7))
 (segment (start 161.798 101.346) (end 148.59 101.346) (width 1) (layer B.Cu) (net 7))
 (segment (start 142.367 95.758) (end 137.541 100.584) (width 1) (layer B.Cu) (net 7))
 (segment (start 143.002 95.758) (end 142.367 95.758) (width 1) (layer B.Cu) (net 7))
 (segment (start 137.541 103.331) (end 139.7 105.49) (width 1) (layer B.Cu) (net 7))
 (segment (start 137.541 100.584) (end 137.541 103.331) (width 1) (layer B.Cu) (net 7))
 (segment (start 132.889 105.49) (end 131.318 107.061) (width 1) (layer B.Cu) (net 7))
 (segment (start 139.7 105.49) (end 132.889 105.49) (width 1) (layer B.Cu) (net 7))
 (segment (start 162.030999 101.346) (end 161.798 101.346) (width 1.5) (layer B.Cu) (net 7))
 (segment (start 173.570001 89.806998) (end 162.030999 101.346) (width 1.5) (layer B.Cu) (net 7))
 (segment (start 157.148991 70.612) (end 157.099 70.612) (width 1.5) (layer B.Cu) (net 7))
 (segment (start 157.099 68.961) (end 160.909 65.151) (width 1) (layer B.Cu) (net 7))
 (segment (start 157.099 70.612) (end 157.099 68.961) (width 1) (layer B.Cu) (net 7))
 (segment (start 173.570001 89.085001) (end 173.570001 89.806998) (width 2) (layer B.Cu) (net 7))
 (segment (start 157.099 72.614) (end 173.570001 89.085001) (width 2) (layer B.Cu) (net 7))
 (segment (start 157.099 70.612) (end 157.099 72.614) (width 2) (layer B.Cu) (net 7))
 (segment (start 117.602 104.14) (end 122.428 99.314) (width 1.5) (layer B.Cu) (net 5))
 (segment (start 117.602 106.847) (end 117.602 104.14) (width 1.5) (layer B.Cu) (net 5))
 (segment (start 122.428 97.038) (end 126.873 92.593) (width 1.5) (layer B.Cu) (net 5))
 (segment (start 122.428 99.314) (end 122.428 97.038) (width 1.5) (layer B.Cu) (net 5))
 (segment (start 164.211 60.833) (end 160.909 57.531) (width 1.5) (layer B.Cu) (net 17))
 (segment (start 164.211 65.151) (end 164.211 60.833) (width 1.5) (layer B.Cu) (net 17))
 (segment (start 160.909 57.531) (end 157.607 57.531) (width 1.5) (layer B.Cu) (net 17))
 (segment (start 164.211 60.833) (end 164.211 60.452) (width 1.5) (layer B.Cu) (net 17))
 (segment (start 167.259 57.404) (end 169.037 57.404) (width 1.5) (layer B.Cu) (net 17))
 (segment (start 164.211 60.452) (end 167.259 57.404) (width 1.5) (layer B.Cu) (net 17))
 (segment (start 108.331 84.963) (end 113.792 90.424) (width 1) (layer B.Cu) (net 4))
 (segment (start 107.188 84.963) (end 108.331 84.963) (width 1) (layer B.Cu) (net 4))
 (segment (start 120.142 90.424) (end 120.57975 89.98625) (width 1) (layer B.Cu) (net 4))
 (segment (start 113.792 90.424) (end 120.142 90.424) (width 1) (layer B.Cu) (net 4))
 (segment (start 137.541 91.104998) (end 137.541 92.964) (width 1) (layer B.Cu) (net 4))
 (segment (start 132.110249 87.786249) (end 134.222251 87.786249) (width 1) (layer B.Cu) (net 4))
 (segment (start 129.910248 89.98625) (end 132.110249 87.786249) (width 1) (layer B.Cu) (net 4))
 (segment (start 134.222251 87.786249) (end 137.541 91.104998) (width 1) (layer B.Cu) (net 4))
 (segment (start 120.57975 89.98625) (end 129.910248 89.98625) (width 1) (layer B.Cu) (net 4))
 (segment (start 140.716 92.964) (end 143.002 90.678) (width 1) (layer B.Cu) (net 4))
 (segment (start 137.541 92.964) (end 140.716 92.964) (width 1) (layer B.Cu) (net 4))
 (segment (start 179.173001 81.303999) (end 179.07 81.407) (width 1) (layer F.Cu) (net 11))
 (segment (start 179.173001 55.540999) (end 179.173001 81.303999) (width 1) (layer F.Cu) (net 11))
 (segment (start 175.372001 51.739999) (end 179.173001 55.540999) (width 1) (layer F.Cu) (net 11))
 (segment (start 126.568001 51.739999) (end 175.372001 51.739999) (width 1) (layer F.Cu) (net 11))
 (segment (start 123.825 54.483) (end 126.568001 51.739999) (width 1) (layer F.Cu) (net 11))
 (segment (start 145.811997 54.940001) (end 146.776998 53.975) (width 1) (layer B.Cu) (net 14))
 (segment (start 144.011999 54.940001) (end 145.811997 54.940001) (width 1) (layer B.Cu) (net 14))
 (segment (start 143.311997 54.239999) (end 144.011999 54.940001) (width 1) (layer B.Cu) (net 14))
 (segment (start 141.511999 54.239999) (end 143.311997 54.239999) (width 1) (layer B.Cu) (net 14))
 (segment (start 133.648998 62.103) (end 141.511999 54.239999) (width 1) (layer B.Cu) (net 14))
 (segment (start 116.713 62.103) (end 133.648998 62.103) (width 1) (layer B.Cu) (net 14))
 (segment (start 113.03 58.42) (end 116.713 62.103) (width 1) (layer B.Cu) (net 14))
 (segment (start 180.975 74.002001) (end 173.570001 81.407) (width 1) (layer B.Cu) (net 14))
 (segment (start 113.03 54.483) (end 113.03 58.42) (width 1) (layer B.Cu) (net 14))
 (segment (start 180.975 64.962998) (end 180.975 74.002001) (width 1) (layer B.Cu) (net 14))
 (segment (start 169.987002 53.975) (end 180.975 64.962998) (width 1) (layer B.Cu) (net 14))
 (segment (start 146.776998 53.975) (end 169.987002 53.975) (width 1) (layer B.Cu) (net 14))
 (segment (start 180.920001 75.852997) (end 180.920001 83.756998) (width 1) (layer B.Cu) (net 12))
 (segment (start 183.515 73.257998) (end 180.920001 75.852997) (width 1) (layer B.Cu) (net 12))
 (segment (start 180.920001 83.756998) (end 179.07 85.606999) (width 1) (layer B.Cu) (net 12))
 (segment (start 134.747 54.483) (end 137.490001 51.739999) (width 1) (layer B.Cu) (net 12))
 (segment (start 183.515 59.882998) (end 183.515 73.257998) (width 1) (layer B.Cu) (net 12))
 (segment (start 175.372001 51.739999) (end 183.515 59.882998) (width 1) (layer B.Cu) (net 12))
 (segment (start 137.490001 51.739999) (end 175.372001 51.739999) (width 1) (layer B.Cu) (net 12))
 (segment (start 122.682 112.268) (end 122.682 111.927) (width 1) (layer B.Cu) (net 13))
 (segment (start 179.07 94.006998) (end 158.522998 114.554) (width 1.5) (layer B.Cu) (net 13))
 (segment (start 124.968 114.554) (end 122.428 112.014) (width 1.5) (layer B.Cu) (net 13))
 (segment (start 158.522998 114.554) (end 124.968 114.554) (width 1.5) (layer B.Cu) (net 13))
 (segment (start 113.919 112.014) (end 107.188 105.283) (width 1) (layer B.Cu) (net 18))
 (segment (start 113.919 114.046) (end 113.919 112.014) (width 1) (layer B.Cu) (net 18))
 (segment (start 150.368 81.28) (end 148.209 83.439) (width 1) (layer B.Cu) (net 9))
 (segment (start 151.765 81.28) (end 150.368 81.28) (width 1) (layer B.Cu) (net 9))
 (segment (start 148.209 90.551) (end 145.542 93.218) (width 1) (layer B.Cu) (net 8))
 (segment (start 148.209 88.519) (end 148.209 90.551) (width 1) (layer B.Cu) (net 8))
 (segment (start 157.848002 81.026) (end 161.798 81.026) (width 1) (layer B.Cu) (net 8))
 (segment (start 150.355002 88.519) (end 157.848002 81.026) (width 1) (layer B.Cu) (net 8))
 (segment (start 148.209 88.519) (end 150.355002 88.519) (width 1) (layer B.Cu) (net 8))
 (segment (start 145.542 93.218) (end 143.002 93.218) (width 1) (layer B.Cu) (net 8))
 (segment (start 151.514991 67.687009) (end 151.514991 76.2) (width 2) (layer B.Cu) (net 16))
 (segment (start 154.051 65.151) (end 151.514991 67.687009) (width 2) (layer B.Cu) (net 16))
 (segment (start 154.051 62.611) (end 147.298087 55.858087) (width 2) (layer B.Cu) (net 16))
 (segment (start 154.051 65.151) (end 154.051 62.611) (width 2) (layer B.Cu) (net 16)))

